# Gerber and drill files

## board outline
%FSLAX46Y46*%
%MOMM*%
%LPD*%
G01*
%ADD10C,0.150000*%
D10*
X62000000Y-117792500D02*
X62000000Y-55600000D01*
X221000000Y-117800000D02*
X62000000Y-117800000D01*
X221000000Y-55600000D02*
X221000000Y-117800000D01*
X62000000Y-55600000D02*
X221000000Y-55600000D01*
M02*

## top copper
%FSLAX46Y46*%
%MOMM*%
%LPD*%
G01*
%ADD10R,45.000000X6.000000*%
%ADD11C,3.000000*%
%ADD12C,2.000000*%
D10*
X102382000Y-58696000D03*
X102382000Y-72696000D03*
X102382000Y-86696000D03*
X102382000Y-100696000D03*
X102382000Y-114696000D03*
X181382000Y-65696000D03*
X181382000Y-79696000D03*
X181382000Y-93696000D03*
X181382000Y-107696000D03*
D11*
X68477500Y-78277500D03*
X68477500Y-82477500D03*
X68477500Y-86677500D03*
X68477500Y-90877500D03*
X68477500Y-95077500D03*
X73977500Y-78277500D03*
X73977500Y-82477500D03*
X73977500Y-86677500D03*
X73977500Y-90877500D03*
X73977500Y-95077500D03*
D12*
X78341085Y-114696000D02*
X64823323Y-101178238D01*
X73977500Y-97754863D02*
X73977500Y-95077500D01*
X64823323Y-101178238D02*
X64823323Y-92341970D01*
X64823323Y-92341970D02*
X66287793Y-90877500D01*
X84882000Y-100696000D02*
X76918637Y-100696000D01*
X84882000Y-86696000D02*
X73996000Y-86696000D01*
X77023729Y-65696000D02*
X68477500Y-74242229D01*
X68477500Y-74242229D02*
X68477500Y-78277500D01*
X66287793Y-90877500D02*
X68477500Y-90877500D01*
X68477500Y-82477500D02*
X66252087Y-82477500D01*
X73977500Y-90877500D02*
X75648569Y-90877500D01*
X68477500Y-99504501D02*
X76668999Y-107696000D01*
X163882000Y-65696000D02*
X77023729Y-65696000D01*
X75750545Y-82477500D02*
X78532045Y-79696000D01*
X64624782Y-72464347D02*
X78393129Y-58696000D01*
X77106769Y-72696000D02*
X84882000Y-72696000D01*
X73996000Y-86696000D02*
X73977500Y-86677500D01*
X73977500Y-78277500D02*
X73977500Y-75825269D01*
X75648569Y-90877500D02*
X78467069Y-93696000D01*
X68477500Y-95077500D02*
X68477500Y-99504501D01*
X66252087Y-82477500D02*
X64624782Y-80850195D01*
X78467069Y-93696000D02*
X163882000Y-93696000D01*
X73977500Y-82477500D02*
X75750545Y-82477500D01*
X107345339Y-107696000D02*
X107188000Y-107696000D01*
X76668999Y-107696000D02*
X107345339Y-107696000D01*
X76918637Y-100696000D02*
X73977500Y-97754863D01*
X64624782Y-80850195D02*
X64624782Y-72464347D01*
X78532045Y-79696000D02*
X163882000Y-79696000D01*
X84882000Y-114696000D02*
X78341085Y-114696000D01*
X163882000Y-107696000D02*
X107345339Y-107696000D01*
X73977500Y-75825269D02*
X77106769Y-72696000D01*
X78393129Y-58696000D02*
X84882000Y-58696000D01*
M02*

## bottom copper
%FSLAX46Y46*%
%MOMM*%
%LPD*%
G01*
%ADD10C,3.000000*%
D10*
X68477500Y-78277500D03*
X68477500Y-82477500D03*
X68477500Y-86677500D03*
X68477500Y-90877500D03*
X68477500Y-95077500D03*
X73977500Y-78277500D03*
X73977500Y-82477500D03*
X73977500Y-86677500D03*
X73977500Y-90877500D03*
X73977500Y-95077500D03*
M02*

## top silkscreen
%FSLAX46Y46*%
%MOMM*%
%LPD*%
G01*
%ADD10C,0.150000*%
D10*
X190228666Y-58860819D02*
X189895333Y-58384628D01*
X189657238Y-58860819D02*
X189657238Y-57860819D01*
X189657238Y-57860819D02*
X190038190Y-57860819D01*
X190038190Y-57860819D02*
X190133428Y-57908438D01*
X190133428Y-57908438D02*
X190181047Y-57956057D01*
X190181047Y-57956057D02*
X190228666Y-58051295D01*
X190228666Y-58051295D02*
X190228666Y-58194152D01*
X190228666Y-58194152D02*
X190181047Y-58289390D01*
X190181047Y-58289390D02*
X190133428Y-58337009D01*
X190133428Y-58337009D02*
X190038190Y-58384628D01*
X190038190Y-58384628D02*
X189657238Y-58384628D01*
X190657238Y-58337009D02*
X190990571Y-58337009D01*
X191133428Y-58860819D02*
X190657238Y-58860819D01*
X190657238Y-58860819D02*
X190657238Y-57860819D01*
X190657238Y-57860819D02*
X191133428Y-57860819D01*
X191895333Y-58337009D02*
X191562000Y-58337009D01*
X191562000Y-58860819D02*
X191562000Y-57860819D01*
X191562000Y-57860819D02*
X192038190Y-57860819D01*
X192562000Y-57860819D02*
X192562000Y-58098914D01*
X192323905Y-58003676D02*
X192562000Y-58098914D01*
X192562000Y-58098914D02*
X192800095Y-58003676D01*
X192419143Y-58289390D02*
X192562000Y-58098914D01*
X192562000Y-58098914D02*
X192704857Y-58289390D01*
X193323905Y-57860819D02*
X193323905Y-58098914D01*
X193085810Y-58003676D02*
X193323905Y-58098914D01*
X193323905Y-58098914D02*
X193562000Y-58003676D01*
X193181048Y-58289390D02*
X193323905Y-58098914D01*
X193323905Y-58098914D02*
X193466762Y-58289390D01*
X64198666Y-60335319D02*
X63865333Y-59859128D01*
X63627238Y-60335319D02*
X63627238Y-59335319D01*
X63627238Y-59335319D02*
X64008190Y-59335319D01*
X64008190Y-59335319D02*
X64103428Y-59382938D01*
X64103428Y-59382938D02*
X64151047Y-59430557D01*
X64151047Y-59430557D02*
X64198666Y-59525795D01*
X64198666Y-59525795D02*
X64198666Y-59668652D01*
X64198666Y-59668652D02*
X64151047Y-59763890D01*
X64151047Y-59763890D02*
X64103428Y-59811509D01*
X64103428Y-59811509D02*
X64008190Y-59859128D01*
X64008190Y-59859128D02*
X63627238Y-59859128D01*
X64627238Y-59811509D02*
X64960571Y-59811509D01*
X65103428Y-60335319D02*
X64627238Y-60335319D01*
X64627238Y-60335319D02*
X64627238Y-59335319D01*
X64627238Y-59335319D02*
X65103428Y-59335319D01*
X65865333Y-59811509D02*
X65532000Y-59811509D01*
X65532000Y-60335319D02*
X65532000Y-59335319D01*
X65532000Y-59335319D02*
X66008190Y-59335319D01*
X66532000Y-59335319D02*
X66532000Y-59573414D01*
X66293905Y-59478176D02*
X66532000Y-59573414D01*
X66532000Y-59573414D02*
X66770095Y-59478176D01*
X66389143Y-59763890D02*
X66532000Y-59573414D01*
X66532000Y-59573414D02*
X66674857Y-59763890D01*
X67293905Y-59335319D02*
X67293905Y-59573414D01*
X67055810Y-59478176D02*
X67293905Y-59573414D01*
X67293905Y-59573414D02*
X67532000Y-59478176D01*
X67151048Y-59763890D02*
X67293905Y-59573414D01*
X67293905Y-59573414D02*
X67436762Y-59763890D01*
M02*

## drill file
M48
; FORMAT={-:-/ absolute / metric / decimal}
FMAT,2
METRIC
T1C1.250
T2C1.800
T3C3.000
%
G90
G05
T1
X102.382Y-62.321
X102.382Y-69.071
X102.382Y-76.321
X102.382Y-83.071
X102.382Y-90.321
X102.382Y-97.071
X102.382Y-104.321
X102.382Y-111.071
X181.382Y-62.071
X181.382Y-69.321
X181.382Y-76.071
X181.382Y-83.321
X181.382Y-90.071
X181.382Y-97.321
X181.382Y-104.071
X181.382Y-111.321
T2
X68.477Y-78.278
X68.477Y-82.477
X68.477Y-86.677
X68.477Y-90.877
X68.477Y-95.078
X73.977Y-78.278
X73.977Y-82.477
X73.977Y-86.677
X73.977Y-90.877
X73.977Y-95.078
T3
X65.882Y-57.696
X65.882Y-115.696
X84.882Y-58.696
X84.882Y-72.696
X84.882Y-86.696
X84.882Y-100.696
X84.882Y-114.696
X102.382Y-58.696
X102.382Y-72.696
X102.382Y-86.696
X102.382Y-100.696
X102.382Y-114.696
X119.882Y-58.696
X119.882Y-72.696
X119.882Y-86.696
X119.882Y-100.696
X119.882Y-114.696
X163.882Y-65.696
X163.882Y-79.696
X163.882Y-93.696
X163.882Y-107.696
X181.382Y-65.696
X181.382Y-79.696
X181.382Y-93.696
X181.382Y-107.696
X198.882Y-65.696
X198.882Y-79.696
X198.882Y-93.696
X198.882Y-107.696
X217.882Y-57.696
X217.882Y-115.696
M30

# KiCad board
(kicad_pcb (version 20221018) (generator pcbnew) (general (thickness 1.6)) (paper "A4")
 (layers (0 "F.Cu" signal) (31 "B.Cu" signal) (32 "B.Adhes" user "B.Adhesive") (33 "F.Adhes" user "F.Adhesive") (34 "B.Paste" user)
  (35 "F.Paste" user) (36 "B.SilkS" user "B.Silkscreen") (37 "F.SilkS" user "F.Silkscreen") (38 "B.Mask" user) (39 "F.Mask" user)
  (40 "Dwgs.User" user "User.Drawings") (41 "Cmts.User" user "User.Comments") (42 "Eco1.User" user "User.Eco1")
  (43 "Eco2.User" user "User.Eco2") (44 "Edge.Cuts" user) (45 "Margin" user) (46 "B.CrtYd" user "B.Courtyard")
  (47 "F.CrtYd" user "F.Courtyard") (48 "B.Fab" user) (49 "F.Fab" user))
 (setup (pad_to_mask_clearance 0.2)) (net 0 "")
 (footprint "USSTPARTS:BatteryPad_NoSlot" (layer "F.Cu") (at 102.382 100.696)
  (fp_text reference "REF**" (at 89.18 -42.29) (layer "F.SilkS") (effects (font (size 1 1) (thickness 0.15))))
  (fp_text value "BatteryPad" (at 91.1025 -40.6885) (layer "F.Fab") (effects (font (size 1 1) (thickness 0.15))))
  (pad "" np_thru_hole circle (at -36.5 -43) (size 3 3) (drill 3) (layers "*.Cu"))
  (pad "" np_thru_hole circle (at -36.5 15) (size 3 3) (drill 3) (layers "*.Cu"))
  (pad "" np_thru_hole circle (at -17.5 -42) (size 3 3) (drill 3) (layers "*.Cu"))
  (pad "" np_thru_hole circle (at -17.5 -28) (size 3 3) (drill 3) (layers "*.Cu"))
  (pad "" np_thru_hole circle (at -17.5 -14) (size 3 3) (drill 3) (layers "*.Cu"))
  (pad "" np_thru_hole circle (at -17.5 0) (size 3 3) (drill 3) (layers "*.Cu"))
  (pad "" np_thru_hole circle (at -17.5 14) (size 3 3) (drill 3) (layers "*.Cu"))
  (pad "" np_thru_hole circle (at 0 -42) (size 3 3) (drill 3) (layers "*.Cu"))
  (pad "" np_thru_hole oval (at 0 -38.375) (size 1.25 1.25) (drill oval 1.25) (layers "*.Cu"))
  (pad "" np_thru_hole oval (at 0 -31.625) (size 1.25 1.25) (drill oval 1.25) (layers "*.Cu"))
  (pad "" np_thru_hole circle (at 0 -28) (size 3 3) (drill 3) (layers "*.Cu"))
  (pad "" np_thru_hole oval (at 0 -24.375) (size 1.25 1.25) (drill oval 1.25) (layers "*.Cu"))
  (pad "" np_thru_hole oval (at 0 -17.625) (size 1.25 1.25) (drill oval 1.25) (layers "*.Cu"))
  (pad "" np_thru_hole circle (at 0 -14) (size 3 3) (drill 3) (layers "*.Cu"))
  (pad "" np_thru_hole oval (at 0 -10.375) (size 1.25 1.25) (drill oval 1.25) (layers "*.Cu"))
  (pad "" np_thru_hole oval (at 0 -3.625) (size 1.25 1.25) (drill oval 1.25) (layers "*.Cu"))
  (pad "" np_thru_hole circle (at 0 0) (size 3 3) (drill 3) (layers "*.Cu"))
  (pad "" np_thru_hole oval (at 0 3.625) (size 1.25 1.25) (drill oval 1.25) (layers "*.Cu"))
  (pad "" np_thru_hole oval (at 0 10.375) (size 1.25 1.25) (drill oval 1.25) (layers "*.Cu"))
  (pad "" np_thru_hole circle (at 0 14) (size 3 3) (drill 3) (layers "*.Cu"))
  (pad "" np_thru_hole circle (at 17.5 -42) (size 3 3) (drill 3) (layers "*.Cu"))
  (pad "" np_thru_hole circle (at 17.5 -28) (size 3 3) (drill 3) (layers "*.Cu"))
  (pad "" np_thru_hole circle (at 17.5 -14) (size 3 3) (drill 3) (layers "*.Cu"))
  (pad "" np_thru_hole circle (at 17.5 0) (size 3 3) (drill 3) (layers "*.Cu"))
  (pad "" np_thru_hole circle (at 17.5 14) (size 3 3) (drill 3) (layers "*.Cu"))
  (pad "" np_thru_hole circle (at 61.5 -35) (size 3 3) (drill 3) (layers "*.Cu"))
  (pad "" np_thru_hole circle (at 61.5 -21) (size 3 3) (drill 3) (layers "*.Cu"))
  (pad "" np_thru_hole circle (at 61.5 -7) (size 3 3) (drill 3) (layers "*.Cu"))
  (pad "" np_thru_hole circle (at 61.5 7) (size 3 3) (drill 3) (layers "*.Cu"))
  (pad "" np_thru_hole oval (at 79 -38.625) (size 1.25 1.25) (drill oval 1.25) (layers "*.Cu"))
  (pad "" np_thru_hole circle (at 79 -35) (size 3 3) (drill 3) (layers "*.Cu"))
  (pad "" np_thru_hole oval (at 79 -31.375) (size 1.25 1.25) (drill oval 1.25) (layers "*.Cu"))
  (pad "" np_thru_hole oval (at 79 -24.625) (size 1.25 1.25) (drill oval 1.25) (layers "*.Cu"))
  (pad "" np_thru_hole circle (at 79 -21) (size 3 3) (drill 3) (layers "*.Cu"))
  (pad "" np_thru_hole oval (at 79 -17.375) (size 1.25 1.25) (drill oval 1.25) (layers "*.Cu"))
  (pad "" np_thru_hole oval (at 79 -10.625) (size 1.25 1.25) (drill oval 1.25) (layers "*.Cu"))
  (pad "" np_thru_hole circle (at 79 -7) (size 3 3) (drill 3) (layers "*.Cu"))
  (pad "" np_thru_hole oval (at 79 -3.375) (size 1.25 1.25) (drill oval 1.25) (layers "*.Cu"))
  (pad "" np_thru_hole oval (at 79 3.375) (size 1.25 1.25) (drill oval 1.25) (layers "*.Cu"))
  (pad "" np_thru_hole circle (at 79 7) (size 3 3) (drill 3) (layers "*.Cu"))
  (pad "" np_thru_hole oval (at 79 10.625) (size 1.25 1.25) (drill oval 1.25) (layers "*.Cu"))
  (pad "" np_thru_hole circle (at 96.5 -35) (size 3 3) (drill 3) (layers "*.Cu"))
  (pad "" np_thru_hole circle (at 96.5 -21) (size 3 3) (drill 3) (layers "*.Cu"))
  (pad "" np_thru_hole circle (at 96.5 -7) (size 3 3) (drill 3) (layers "*.Cu"))
  (pad "" np_thru_hole circle (at 96.5 7) (size 3 3) (drill 3) (layers "*.Cu"))
  (pad "" np_thru_hole circle (at 115.5 -43) (size 3 3) (drill 3) (layers "*.Cu"))
  (pad "" np_thru_hole circle (at 115.5 15) (size 3 3) (drill 3) (layers "*.Cu")) (pad "1" smd rect (at 0 -42) (size 45 6) (layers "F.Cu"))
  (pad "1" smd rect (at 0 -28) (size 45 6) (layers "F.Cu")) (pad "1" smd rect (at 0 -14) (size 45 6) (layers "F.Cu"))
  (pad "1" smd rect (at 0 0) (size 45 6) (layers "F.Cu")) (pad "1" smd rect (at 0 14) (size 45 6) (layers "F.Cu"))
  (pad "1" smd rect (at 79 -35) (size 45 6) (layers "F.Cu")) (pad "1" smd rect (at 79 -21) (size 45 6) (layers "F.Cu"))
  (pad "1" smd rect (at 79 -7) (size 45 6) (layers "F.Cu")) (pad "1" smd rect (at 79 7) (size 45 6) (layers "F.Cu")))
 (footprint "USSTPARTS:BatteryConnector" (layer "F.Cu") (at 68.4775 95.0775)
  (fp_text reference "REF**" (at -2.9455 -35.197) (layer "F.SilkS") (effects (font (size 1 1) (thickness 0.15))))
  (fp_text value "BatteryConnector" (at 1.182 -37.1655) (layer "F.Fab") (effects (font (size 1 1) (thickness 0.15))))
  (pad "" np_thru_hole circle (at 0 -16.8) (size 3 3) (drill 1.8) (layers "*.Cu"))
  (pad "" np_thru_hole circle (at 0 -12.6) (size 3 3) (drill 1.8) (layers "*.Cu"))
  (pad "" np_thru_hole circle (at 0 -8.4) (size 3 3) (drill 1.8) (layers "*.Cu"))
  (pad "" np_thru_hole circle (at 0 -4.2) (size 3 3) (drill 1.8) (layers "*.Cu"))
  (pad "" np_thru_hole circle (at 0 0) (size 3 3) (drill 1.8) (layers "*.Cu"))
  (pad "" np_thru_hole circle (at 5.5 -16.8) (size 3 3) (drill 1.8) (layers "*.Cu"))
  (pad "" np_thru_hole circle (at 5.5 -12.6) (size 3 3) (drill 1.8) (layers "*.Cu"))
  (pad "" np_thru_hole circle (at 5.5 -8.4) (size 3 3) (drill 1.8) (layers "*.Cu"))
  (pad "" np_thru_hole circle (at 5.5 -4.2) (size 3 3) (drill 1.8) (layers "*.Cu"))
  (pad "" np_thru_hole circle (at 5.5 0) (size 3 3) (drill 1.8) (layers "*.Cu")))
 (gr_line (start 62 117.7925) (end 62 55.6) (stroke (width 0.15) (type solid)) (layer "Edge.Cuts"))
 (gr_line (start 221 117.8) (end 62 117.8) (stroke (width 0.15) (type solid)) (layer "Edge.Cuts"))
 (gr_line (start 221 55.6) (end 221 117.8) (stroke (width 0.15) (type solid)) (layer "Edge.Cuts"))
 (gr_line (start 62 55.6) (end 221 55.6) (stroke (width 0.15) (type solid)) (layer "Edge.Cuts"))
 (segment (start 78.341085 114.696) (end 64.823323 101.178238) (width 2) (layer "F.Cu") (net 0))
 (segment (start 73.9775 97.754863) (end 73.9775 95.0775) (width 2) (layer "F.Cu") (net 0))
 (segment (start 64.823323 101.178238) (end 64.823323 92.34197) (width 2) (layer "F.Cu") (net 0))
 (segment (start 64.823323 92.34197) (end 66.287793 90.8775) (width 2) (layer "F.Cu") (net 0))
 (segment (start 84.882 100.696) (end 76.918637 100.696) (width 2) (layer "F.Cu") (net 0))
 (segment (start 84.882 86.696) (end 73.996 86.696) (width 2) (layer "F.Cu") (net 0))
 (segment (start 77.023729 65.696) (end 68.4775 74.242229) (width 2) (layer "F.Cu") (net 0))
 (segment (start 68.4775 74.242229) (end 68.4775 78.2775) (width 2) (layer "F.Cu") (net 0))
 (segment (start 66.287793 90.8775) (end 68.4775 90.8775) (width 2) (layer "F.Cu") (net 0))
 (segment (start 68.4775 82.4775) (end 66.252087 82.4775) (width 2) (layer "F.Cu") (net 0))
 (segment (start 73.9775 90.8775) (end 75.648569 90.8775) (width 2) (layer "F.Cu") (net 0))
 (segment (start 68.4775 99.504501) (end 76.668999 107.696) (width 2) (layer "F.Cu") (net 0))
 (segment (start 163.882 65.696) (end 77.023729 65.696) (width 2) (layer "F.Cu") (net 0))
 (segment (start 75.750545 82.4775) (end 78.532045 79.696) (width 2) (layer "F.Cu") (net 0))
 (segment (start 64.624782 72.464347) (end 78.393129 58.696) (width 2) (layer "F.Cu") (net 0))
 (segment (start 77.106769 72.696) (end 84.882 72.696) (width 2) (layer "F.Cu") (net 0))
 (segment (start 73.996 86.696) (end 73.9775 86.6775) (width 2) (layer "F.Cu") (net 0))
 (segment (start 73.9775 78.2775) (end 73.9775 75.825269) (width 2) (layer "F.Cu") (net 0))
 (segment (start 75.648569 90.8775) (end 78.467069 93.696) (width 2) (layer "F.Cu") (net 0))
 (segment (start 68.4775 95.0775) (end 68.4775 99.504501) (width 2) (layer "F.Cu") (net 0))
 (segment (start 66.252087 82.4775) (end 64.624782 80.850195) (width 2) (layer "F.Cu") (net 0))
 (segment (start 78.467069 93.696) (end 163.882 93.696) (width 2) (layer "F.Cu") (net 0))
 (segment (start 73.9775 82.4775) (end 75.750545 82.4775) (width 2) (layer "F.Cu") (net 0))
 (segment (start 107.345339 107.696) (end 107.188 107.696) (width 2) (layer "F.Cu") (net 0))
 (segment (start 76.668999 107.696) (end 107.345339 107.696) (width 2) (layer "F.Cu") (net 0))
 (segment (start 76.918637 100.696) (end 73.9775 97.754863) (width 2) (layer "F.Cu") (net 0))
 (segment (start 64.624782 80.850195) (end 64.624782 72.464347) (width 2) (layer "F.Cu") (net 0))
 (segment (start 78.532045 79.696) (end 163.882 79.696) (width 2) (layer "F.Cu") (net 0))
 (segment (start 84.882 114.696) (end 78.341085 114.696) (width 2) (layer "F.Cu") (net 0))
 (segment (start 163.882 107.696) (end 107.345339 107.696) (width 2) (layer "F.Cu") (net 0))
 (segment (start 73.9775 75.825269) (end 77.106769 72.696) (width 2) (layer "F.Cu") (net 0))
 (segment (start 78.393129 58.696) (end 84.882 58.696) (width 2) (layer "F.Cu") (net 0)))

